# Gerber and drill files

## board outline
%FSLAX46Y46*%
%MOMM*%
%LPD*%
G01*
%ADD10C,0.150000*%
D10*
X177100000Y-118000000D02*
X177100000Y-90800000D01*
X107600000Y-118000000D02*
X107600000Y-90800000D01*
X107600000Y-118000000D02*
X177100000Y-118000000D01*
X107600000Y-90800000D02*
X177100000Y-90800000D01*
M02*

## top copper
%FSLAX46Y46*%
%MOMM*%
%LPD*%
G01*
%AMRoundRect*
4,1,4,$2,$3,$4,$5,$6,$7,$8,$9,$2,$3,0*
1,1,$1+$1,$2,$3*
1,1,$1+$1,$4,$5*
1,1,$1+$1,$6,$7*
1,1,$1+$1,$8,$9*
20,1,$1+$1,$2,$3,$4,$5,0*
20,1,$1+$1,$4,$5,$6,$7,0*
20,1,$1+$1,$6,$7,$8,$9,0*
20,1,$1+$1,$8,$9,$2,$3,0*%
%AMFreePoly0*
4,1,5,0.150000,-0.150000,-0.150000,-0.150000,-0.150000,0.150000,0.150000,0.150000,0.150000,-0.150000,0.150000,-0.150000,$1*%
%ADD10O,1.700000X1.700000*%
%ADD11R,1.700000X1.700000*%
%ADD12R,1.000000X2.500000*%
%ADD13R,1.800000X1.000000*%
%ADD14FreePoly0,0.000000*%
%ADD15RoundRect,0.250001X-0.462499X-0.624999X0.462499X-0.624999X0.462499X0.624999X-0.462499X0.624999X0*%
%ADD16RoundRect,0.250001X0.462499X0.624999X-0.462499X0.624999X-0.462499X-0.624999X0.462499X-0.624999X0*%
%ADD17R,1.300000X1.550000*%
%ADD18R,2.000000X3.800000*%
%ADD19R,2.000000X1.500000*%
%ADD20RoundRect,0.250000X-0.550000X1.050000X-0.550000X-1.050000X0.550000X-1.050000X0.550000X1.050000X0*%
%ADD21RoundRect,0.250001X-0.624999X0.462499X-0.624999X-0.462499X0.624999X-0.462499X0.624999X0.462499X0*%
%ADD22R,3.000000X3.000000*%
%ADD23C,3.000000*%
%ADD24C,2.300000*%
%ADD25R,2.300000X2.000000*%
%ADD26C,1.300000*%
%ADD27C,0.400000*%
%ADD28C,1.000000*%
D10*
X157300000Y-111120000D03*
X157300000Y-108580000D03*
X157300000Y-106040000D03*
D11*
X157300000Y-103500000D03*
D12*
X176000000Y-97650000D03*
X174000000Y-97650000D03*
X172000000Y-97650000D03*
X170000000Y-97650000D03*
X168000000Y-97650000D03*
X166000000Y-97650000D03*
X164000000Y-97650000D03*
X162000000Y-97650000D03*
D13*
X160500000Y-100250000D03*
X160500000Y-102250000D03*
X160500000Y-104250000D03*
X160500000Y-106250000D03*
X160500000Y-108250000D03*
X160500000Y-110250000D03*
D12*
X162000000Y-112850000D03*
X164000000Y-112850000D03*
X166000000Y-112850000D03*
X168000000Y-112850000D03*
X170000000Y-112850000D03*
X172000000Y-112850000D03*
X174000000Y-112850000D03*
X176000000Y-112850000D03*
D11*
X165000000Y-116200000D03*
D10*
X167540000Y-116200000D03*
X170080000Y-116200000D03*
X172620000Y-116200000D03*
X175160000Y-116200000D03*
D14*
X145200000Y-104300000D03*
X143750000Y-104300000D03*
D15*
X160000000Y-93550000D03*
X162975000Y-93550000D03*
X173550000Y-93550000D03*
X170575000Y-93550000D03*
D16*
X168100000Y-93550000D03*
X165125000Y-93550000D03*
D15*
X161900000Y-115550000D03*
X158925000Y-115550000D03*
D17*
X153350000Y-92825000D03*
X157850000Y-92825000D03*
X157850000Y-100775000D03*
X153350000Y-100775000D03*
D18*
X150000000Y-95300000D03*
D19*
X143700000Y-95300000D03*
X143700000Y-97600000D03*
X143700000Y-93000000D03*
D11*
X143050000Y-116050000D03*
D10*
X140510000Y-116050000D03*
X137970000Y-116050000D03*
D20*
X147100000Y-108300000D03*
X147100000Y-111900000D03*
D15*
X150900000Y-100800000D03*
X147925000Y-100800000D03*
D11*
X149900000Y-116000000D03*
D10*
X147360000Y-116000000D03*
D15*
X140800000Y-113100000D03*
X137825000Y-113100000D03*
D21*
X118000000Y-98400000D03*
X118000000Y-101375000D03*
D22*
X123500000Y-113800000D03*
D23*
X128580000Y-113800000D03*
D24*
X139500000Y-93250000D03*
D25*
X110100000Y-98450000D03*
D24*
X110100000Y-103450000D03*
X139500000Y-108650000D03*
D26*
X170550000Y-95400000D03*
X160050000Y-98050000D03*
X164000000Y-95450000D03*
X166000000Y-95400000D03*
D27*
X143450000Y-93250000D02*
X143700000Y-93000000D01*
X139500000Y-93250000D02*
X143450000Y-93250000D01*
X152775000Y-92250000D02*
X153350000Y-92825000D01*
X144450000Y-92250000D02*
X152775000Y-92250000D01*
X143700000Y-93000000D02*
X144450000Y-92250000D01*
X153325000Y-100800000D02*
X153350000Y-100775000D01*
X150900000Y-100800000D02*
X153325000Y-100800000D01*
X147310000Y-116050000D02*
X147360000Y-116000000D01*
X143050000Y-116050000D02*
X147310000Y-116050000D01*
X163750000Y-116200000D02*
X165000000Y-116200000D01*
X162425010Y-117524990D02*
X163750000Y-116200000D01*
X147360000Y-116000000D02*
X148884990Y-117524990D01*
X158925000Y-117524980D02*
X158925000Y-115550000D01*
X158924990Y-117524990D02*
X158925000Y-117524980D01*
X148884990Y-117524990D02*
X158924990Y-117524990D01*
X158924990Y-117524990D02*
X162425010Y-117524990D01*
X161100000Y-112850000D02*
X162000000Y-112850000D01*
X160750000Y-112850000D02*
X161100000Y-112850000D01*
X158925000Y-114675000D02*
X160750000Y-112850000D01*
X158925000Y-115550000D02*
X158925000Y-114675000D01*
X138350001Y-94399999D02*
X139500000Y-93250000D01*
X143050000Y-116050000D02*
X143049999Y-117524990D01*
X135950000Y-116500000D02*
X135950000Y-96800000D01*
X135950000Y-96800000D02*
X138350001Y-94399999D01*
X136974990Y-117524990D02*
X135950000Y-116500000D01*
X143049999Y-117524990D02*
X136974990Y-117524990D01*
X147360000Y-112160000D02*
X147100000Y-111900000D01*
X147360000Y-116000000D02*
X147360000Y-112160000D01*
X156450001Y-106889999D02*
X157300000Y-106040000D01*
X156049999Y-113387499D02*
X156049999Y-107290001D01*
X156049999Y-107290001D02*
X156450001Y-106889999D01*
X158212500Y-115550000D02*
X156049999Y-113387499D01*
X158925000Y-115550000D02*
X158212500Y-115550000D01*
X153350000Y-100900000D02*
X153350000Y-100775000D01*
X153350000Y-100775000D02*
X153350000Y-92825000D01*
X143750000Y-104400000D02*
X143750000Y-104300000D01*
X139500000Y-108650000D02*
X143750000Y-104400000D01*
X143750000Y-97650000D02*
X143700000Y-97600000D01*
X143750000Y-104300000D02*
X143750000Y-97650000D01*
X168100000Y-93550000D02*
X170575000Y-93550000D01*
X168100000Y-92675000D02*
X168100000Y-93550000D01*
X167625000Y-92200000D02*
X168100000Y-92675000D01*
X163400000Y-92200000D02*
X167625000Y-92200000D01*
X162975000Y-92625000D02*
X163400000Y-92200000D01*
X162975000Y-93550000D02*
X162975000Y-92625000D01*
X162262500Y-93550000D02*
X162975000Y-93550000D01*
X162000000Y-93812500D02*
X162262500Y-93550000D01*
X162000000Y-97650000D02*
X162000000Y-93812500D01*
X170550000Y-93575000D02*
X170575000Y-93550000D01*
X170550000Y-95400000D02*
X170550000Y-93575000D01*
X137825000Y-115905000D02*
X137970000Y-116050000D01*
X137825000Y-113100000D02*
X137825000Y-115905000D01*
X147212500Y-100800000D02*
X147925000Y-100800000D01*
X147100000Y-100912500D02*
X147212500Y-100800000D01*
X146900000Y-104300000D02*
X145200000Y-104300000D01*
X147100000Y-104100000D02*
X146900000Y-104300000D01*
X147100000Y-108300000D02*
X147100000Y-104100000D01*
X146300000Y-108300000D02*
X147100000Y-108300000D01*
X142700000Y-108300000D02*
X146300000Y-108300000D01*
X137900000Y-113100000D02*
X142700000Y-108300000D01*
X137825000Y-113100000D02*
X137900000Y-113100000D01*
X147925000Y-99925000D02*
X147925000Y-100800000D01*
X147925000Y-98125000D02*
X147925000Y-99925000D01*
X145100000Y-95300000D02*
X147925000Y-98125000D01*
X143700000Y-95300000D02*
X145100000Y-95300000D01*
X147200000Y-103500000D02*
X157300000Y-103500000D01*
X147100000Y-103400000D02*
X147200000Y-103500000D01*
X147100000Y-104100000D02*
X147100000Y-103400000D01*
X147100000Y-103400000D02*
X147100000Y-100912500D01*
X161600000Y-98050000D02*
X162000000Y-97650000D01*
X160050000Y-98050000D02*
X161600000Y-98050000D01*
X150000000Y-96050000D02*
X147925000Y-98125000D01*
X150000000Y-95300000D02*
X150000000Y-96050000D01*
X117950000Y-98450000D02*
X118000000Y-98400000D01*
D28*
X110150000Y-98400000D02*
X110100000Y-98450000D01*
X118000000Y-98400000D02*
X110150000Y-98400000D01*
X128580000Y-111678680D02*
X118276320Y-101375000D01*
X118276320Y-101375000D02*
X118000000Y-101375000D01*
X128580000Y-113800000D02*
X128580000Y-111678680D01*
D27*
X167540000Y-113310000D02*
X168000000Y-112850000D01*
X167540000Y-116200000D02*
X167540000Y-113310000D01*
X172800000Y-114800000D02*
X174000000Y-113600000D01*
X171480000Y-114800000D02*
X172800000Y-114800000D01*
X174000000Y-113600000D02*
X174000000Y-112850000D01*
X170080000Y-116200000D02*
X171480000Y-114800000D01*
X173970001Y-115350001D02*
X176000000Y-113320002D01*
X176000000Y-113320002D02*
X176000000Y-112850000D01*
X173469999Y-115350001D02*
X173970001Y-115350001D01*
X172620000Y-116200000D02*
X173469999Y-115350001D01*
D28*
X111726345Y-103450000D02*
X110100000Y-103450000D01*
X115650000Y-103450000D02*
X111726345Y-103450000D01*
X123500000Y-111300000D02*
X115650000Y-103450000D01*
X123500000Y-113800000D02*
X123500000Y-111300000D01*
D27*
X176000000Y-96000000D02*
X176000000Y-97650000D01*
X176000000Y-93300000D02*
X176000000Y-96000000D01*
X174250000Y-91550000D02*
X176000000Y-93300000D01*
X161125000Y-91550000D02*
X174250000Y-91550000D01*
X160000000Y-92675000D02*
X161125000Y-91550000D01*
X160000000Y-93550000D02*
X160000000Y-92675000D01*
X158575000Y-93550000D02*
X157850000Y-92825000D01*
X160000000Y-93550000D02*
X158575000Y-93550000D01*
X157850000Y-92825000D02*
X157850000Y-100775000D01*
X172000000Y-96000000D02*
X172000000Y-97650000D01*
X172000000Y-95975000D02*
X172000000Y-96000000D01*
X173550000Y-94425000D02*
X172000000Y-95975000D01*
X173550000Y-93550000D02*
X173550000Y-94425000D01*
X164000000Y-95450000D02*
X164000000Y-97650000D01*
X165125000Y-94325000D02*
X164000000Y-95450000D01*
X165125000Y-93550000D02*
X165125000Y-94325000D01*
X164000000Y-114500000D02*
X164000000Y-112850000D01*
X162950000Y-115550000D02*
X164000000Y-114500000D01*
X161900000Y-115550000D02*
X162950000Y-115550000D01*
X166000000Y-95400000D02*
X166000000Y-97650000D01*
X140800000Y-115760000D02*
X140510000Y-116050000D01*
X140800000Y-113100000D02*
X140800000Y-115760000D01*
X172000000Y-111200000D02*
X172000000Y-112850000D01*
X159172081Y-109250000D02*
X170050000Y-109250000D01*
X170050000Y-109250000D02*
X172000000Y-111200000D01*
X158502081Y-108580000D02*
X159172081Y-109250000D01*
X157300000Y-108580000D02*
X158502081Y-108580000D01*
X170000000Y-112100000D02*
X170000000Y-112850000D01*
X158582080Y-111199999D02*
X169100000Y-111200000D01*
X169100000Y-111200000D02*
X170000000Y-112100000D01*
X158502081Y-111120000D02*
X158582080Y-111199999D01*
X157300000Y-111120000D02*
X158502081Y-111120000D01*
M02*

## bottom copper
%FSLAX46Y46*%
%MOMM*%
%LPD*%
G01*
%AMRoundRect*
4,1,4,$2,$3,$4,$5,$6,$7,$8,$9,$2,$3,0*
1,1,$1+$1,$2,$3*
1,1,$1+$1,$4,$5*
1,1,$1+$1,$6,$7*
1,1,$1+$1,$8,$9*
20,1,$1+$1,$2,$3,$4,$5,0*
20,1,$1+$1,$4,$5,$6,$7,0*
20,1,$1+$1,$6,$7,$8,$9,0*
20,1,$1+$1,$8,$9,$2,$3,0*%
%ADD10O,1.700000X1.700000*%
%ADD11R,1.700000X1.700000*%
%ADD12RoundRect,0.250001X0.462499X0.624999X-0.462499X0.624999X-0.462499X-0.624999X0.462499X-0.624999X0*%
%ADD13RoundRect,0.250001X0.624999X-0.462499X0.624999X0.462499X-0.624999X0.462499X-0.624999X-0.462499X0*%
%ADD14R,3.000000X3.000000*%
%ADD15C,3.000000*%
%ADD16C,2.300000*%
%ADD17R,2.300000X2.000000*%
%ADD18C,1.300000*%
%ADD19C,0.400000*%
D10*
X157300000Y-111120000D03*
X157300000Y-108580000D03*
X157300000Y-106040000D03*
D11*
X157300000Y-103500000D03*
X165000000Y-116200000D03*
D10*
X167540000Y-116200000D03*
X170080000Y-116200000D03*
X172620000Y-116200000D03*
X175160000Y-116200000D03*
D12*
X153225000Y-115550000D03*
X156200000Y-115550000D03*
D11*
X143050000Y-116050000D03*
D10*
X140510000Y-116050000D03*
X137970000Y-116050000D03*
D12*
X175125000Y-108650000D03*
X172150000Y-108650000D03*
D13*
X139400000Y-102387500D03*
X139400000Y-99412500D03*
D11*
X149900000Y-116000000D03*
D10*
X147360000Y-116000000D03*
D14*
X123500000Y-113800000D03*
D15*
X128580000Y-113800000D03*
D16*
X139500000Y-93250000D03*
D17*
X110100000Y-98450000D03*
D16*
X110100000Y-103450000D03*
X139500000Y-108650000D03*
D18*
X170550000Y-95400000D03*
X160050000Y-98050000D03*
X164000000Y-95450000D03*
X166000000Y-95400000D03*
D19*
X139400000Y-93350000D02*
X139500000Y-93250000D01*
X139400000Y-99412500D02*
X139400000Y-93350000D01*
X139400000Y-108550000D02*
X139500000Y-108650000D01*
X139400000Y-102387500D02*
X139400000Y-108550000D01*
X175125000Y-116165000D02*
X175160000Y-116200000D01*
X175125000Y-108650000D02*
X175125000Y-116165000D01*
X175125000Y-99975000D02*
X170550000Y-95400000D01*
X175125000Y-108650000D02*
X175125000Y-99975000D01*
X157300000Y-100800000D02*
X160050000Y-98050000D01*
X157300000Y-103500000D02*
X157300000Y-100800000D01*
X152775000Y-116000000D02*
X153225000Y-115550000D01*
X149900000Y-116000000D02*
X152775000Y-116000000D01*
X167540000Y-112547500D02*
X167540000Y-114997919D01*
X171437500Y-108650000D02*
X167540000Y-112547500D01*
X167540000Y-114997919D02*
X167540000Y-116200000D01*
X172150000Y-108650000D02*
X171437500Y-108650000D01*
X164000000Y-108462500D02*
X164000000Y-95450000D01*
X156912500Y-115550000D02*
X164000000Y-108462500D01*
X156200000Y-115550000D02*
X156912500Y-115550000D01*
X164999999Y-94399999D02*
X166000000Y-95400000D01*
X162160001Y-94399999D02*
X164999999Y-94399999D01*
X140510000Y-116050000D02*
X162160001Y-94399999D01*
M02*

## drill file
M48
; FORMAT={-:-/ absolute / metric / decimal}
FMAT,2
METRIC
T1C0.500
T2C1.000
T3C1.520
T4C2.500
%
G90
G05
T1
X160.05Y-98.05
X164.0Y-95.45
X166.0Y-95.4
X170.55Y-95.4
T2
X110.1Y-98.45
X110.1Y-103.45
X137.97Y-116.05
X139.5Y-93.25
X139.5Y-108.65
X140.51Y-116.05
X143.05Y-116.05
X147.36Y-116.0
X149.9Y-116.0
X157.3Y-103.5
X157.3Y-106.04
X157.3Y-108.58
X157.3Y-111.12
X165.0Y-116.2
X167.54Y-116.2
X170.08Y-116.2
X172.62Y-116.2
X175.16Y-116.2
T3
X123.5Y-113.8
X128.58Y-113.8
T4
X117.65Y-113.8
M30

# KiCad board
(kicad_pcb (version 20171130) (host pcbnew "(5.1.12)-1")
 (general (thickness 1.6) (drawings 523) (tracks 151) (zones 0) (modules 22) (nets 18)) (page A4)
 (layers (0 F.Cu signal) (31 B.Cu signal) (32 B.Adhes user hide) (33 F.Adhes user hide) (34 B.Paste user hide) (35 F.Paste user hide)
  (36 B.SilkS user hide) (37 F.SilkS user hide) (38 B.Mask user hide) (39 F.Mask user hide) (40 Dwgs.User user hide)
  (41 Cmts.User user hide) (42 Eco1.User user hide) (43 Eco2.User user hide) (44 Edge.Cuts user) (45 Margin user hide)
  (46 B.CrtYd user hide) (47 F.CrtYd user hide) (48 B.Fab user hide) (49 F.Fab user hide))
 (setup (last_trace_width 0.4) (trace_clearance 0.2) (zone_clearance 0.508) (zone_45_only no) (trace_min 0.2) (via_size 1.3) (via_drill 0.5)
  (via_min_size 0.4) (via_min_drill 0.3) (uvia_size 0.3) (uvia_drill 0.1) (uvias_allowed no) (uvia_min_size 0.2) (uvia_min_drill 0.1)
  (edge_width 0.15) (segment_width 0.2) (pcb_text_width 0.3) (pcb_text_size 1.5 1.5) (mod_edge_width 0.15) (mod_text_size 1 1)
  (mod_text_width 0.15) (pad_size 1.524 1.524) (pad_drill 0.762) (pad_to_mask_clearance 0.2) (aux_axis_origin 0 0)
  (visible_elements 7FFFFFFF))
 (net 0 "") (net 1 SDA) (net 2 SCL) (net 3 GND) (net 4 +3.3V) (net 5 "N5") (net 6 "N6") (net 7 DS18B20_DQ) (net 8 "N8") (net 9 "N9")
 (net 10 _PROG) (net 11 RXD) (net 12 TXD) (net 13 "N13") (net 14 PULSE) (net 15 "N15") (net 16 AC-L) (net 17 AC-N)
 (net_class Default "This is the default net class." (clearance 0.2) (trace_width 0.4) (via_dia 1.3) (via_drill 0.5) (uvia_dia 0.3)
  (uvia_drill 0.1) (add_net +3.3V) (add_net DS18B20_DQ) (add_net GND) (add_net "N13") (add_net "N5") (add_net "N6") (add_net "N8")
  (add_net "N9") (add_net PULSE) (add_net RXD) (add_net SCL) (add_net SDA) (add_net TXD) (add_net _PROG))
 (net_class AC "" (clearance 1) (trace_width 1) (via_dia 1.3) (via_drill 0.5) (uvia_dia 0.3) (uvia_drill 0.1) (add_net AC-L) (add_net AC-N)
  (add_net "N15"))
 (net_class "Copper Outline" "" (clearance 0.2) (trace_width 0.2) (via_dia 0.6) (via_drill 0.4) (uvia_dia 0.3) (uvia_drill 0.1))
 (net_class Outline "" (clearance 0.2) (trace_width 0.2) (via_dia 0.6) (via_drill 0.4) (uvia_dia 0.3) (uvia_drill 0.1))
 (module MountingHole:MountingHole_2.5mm (layer F.Cu) (at 117.65 113.8)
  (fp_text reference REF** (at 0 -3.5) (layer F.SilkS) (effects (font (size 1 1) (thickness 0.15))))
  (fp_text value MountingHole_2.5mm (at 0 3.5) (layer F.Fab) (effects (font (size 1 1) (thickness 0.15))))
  (pad 1 np_thru_hole circle (at 0 0) (size 2.5 2.5) (drill 2.5) (layers *.Cu *.Mask)))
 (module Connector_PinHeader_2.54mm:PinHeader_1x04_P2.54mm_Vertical (layer F.Cu) (at 157.3 103.5)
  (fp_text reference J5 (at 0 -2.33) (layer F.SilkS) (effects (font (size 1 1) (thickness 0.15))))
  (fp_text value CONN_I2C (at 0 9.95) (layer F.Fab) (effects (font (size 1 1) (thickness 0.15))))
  (pad 4 thru_hole oval (at 0 7.62) (size 1.7 1.7) (drill 1) (layers *.Cu *.Mask) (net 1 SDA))
  (pad 3 thru_hole oval (at 0 5.08) (size 1.7 1.7) (drill 1) (layers *.Cu *.Mask) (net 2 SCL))
  (pad 2 thru_hole oval (at 0 2.54) (size 1.7 1.7) (drill 1) (layers *.Cu *.Mask) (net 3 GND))
  (pad 1 thru_hole rect (at 0 0) (size 1.7 1.7) (drill 1) (layers *.Cu *.Mask) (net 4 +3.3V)))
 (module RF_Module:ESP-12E (layer F.Cu) (at 172.5 105.25 270)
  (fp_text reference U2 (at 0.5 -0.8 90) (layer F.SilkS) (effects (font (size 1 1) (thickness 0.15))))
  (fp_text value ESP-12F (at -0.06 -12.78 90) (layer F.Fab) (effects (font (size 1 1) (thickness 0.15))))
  (pad 1 smd rect (at -7.6 -3.5 270) (size 2.5 1) (layers F.Cu F.Paste F.Mask) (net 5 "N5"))
  (pad 2 smd rect (at -7.6 -1.5 270) (size 2.5 1) (layers F.Cu F.Paste F.Mask))
  (pad 3 smd rect (at -7.6 0.5 270) (size 2.5 1) (layers F.Cu F.Paste F.Mask) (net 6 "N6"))
  (pad 4 smd rect (at -7.6 2.5 270) (size 2.5 1) (layers F.Cu F.Paste F.Mask))
  (pad 5 smd rect (at -7.6 4.5 270) (size 2.5 1) (layers F.Cu F.Paste F.Mask))
  (pad 6 smd rect (at -7.6 6.5 270) (size 2.5 1) (layers F.Cu F.Paste F.Mask) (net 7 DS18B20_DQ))
  (pad 7 smd rect (at -7.6 8.5 270) (size 2.5 1) (layers F.Cu F.Paste F.Mask) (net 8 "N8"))
  (pad 8 smd rect (at -7.6 10.5 270) (size 2.5 1) (layers F.Cu F.Paste F.Mask) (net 4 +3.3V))
  (pad 9 smd rect (at -5 12 270) (size 1 1.8) (layers F.Cu F.Paste F.Mask))
  (pad 10 smd rect (at -3 12 270) (size 1 1.8) (layers F.Cu F.Paste F.Mask))
  (pad 11 smd rect (at -1 12 270) (size 1 1.8) (layers F.Cu F.Paste F.Mask))
  (pad 12 smd rect (at 1 12 270) (size 1 1.8) (layers F.Cu F.Paste F.Mask))
  (pad 13 smd rect (at 3 12 270) (size 1 1.8) (layers F.Cu F.Paste F.Mask))
  (pad 14 smd rect (at 5 12 270) (size 1 1.8) (layers F.Cu F.Paste F.Mask))
  (pad 15 smd rect (at 7.6 10.5 270) (size 2.5 1) (layers F.Cu F.Paste F.Mask) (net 3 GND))
  (pad 16 smd rect (at 7.6 8.5 270) (size 2.5 1) (layers F.Cu F.Paste F.Mask) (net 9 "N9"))
  (pad 17 smd rect (at 7.6 6.5 270) (size 2.5 1) (layers F.Cu F.Paste F.Mask))
  (pad 18 smd rect (at 7.6 4.5 270) (size 2.5 1) (layers F.Cu F.Paste F.Mask) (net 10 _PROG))
  (pad 19 smd rect (at 7.6 2.5 270) (size 2.5 1) (layers F.Cu F.Paste F.Mask) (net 1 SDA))
  (pad 20 smd rect (at 7.6 0.5 270) (size 2.5 1) (layers F.Cu F.Paste F.Mask) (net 2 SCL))
  (pad 21 smd rect (at 7.6 -1.5 270) (size 2.5 1) (layers F.Cu F.Paste F.Mask) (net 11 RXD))
  (pad 22 smd rect (at 7.6 -3.5 270) (size 2.5 1) (layers F.Cu F.Paste F.Mask) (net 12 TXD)))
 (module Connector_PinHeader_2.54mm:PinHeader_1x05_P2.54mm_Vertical (layer F.Cu) (at 165 116.2 90)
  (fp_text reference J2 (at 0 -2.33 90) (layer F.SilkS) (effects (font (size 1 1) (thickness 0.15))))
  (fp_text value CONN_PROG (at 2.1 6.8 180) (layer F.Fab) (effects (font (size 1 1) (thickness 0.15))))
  (pad 1 thru_hole rect (at 0 0 90) (size 1.7 1.7) (drill 1) (layers *.Cu *.Mask) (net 3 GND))
  (pad 2 thru_hole oval (at 0 2.54 90) (size 1.7 1.7) (drill 1) (layers *.Cu *.Mask) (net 10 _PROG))
  (pad 3 thru_hole oval (at 0 5.08 90) (size 1.7 1.7) (drill 1) (layers *.Cu *.Mask) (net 11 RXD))
  (pad 4 thru_hole oval (at 0 7.62 90) (size 1.7 1.7) (drill 1) (layers *.Cu *.Mask) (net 12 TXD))
  (pad 5 thru_hole oval (at 0 10.16 90) (size 1.7 1.7) (drill 1) (layers *.Cu *.Mask) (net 4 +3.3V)))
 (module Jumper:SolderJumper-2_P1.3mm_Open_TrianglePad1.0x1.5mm (layer F.Cu) (at 144.475 104.3)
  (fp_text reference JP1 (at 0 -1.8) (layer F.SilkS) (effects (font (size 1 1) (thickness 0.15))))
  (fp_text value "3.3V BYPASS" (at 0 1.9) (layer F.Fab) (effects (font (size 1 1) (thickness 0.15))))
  (pad 2 smd custom (at 0.725 0) (size 0.3 0.3) (layers F.Cu F.Mask) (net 4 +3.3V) (zone_connect 2)
   (options (clearance outline) (anchor rect)) (primitives))
  (pad 1 smd custom (at -0.725 0) (size 0.3 0.3) (layers F.Cu F.Mask) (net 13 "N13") (zone_connect 2)
   (options (clearance outline) (anchor rect)) (primitives)))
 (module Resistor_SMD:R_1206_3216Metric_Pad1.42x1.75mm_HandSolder (layer F.Cu) (at 161.4875 93.55)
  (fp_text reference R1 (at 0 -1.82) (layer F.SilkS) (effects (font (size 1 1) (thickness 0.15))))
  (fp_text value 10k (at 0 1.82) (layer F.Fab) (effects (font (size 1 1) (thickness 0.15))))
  (pad 1 smd roundrect (at -1.4875 0) (size 1.425 1.75) (layers F.Cu F.Paste F.Mask) (roundrect_rratio 0.175439) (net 5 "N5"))
  (pad 2 smd roundrect (at 1.4875 0) (size 1.425 1.75) (layers F.Cu F.Paste F.Mask) (roundrect_rratio 0.175439) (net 4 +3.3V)))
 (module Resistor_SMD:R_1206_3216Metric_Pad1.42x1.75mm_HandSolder (layer F.Cu) (at 172.0625 93.55)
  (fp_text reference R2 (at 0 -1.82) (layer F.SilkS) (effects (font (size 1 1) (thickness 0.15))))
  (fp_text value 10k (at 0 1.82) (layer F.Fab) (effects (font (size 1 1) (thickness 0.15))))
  (pad 2 smd roundrect (at 1.4875 0) (size 1.425 1.75) (layers F.Cu F.Paste F.Mask) (roundrect_rratio 0.175439) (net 6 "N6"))
  (pad 1 smd roundrect (at -1.4875 0) (size 1.425 1.75) (layers F.Cu F.Paste F.Mask) (roundrect_rratio 0.175439) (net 4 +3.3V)))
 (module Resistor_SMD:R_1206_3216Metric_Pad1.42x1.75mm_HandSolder (layer B.Cu) (at 154.7125 115.55 180)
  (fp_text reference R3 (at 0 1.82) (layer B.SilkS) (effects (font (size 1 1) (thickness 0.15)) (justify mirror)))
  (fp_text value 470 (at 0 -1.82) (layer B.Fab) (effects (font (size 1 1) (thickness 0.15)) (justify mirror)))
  (pad 2 smd roundrect (at 1.4875 0 180) (size 1.425 1.75) (layers B.Cu B.Paste B.Mask) (roundrect_rratio 0.175439) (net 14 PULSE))
  (pad 1 smd roundrect (at -1.4875 0 180) (size 1.425 1.75) (layers B.Cu B.Paste B.Mask) (roundrect_rratio 0.175439) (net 8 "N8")))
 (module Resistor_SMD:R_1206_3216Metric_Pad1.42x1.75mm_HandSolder (layer F.Cu) (at 166.6125 93.55 180)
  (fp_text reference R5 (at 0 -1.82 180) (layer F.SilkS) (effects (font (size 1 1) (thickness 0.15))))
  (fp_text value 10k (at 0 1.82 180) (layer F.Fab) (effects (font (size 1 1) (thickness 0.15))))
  (pad 1 smd roundrect (at -1.4875 0 180) (size 1.425 1.75) (layers F.Cu F.Paste F.Mask) (roundrect_rratio 0.175439) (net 4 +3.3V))
  (pad 2 smd roundrect (at 1.4875 0 180) (size 1.425 1.75) (layers F.Cu F.Paste F.Mask) (roundrect_rratio 0.175439) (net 8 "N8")))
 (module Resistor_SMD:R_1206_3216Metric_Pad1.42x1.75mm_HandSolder (layer F.Cu) (at 160.4125 115.55)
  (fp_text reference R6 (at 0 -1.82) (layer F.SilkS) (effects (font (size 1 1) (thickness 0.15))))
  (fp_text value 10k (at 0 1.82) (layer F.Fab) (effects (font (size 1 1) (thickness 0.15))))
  (pad 2 smd roundrect (at 1.4875 0) (size 1.425 1.75) (layers F.Cu F.Paste F.Mask) (roundrect_rratio 0.175439) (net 9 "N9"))
  (pad 1 smd roundrect (at -1.4875 0) (size 1.425 1.75) (layers F.Cu F.Paste F.Mask) (roundrect_rratio 0.175439) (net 3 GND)))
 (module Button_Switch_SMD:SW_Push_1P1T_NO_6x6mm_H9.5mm (layer F.Cu) (at 155.6 96.8 270)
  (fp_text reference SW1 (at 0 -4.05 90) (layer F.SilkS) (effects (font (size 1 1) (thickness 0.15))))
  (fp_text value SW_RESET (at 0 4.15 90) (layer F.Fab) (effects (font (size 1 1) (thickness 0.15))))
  (pad 2 smd rect (at -3.975 2.25 270) (size 1.55 1.3) (layers F.Cu F.Paste F.Mask) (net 3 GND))
  (pad 1 smd rect (at -3.975 -2.25 270) (size 1.55 1.3) (layers F.Cu F.Paste F.Mask) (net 5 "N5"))
  (pad 1 smd rect (at 3.975 -2.25 270) (size 1.55 1.3) (layers F.Cu F.Paste F.Mask) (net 5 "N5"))
  (pad 2 smd rect (at 3.975 2.25 270) (size 1.55 1.3) (layers F.Cu F.Paste F.Mask) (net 3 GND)))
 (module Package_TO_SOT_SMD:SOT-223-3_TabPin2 (layer F.Cu) (at 146.85 95.3)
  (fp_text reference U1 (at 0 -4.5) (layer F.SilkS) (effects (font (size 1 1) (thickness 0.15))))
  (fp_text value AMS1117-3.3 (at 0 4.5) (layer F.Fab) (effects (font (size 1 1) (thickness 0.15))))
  (pad 2 smd rect (at 3.15 0) (size 2 3.8) (layers F.Cu F.Paste F.Mask) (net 4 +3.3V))
  (pad 2 smd rect (at -3.15 0) (size 2 1.5) (layers F.Cu F.Paste F.Mask) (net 4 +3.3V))
  (pad 3 smd rect (at -3.15 2.3) (size 2 1.5) (layers F.Cu F.Paste F.Mask) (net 13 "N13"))
  (pad 1 smd rect (at -3.15 -2.3) (size 2 1.5) (layers F.Cu F.Paste F.Mask) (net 3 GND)))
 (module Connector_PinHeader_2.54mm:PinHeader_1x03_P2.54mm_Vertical (layer F.Cu) (at 143.05 116.05 270)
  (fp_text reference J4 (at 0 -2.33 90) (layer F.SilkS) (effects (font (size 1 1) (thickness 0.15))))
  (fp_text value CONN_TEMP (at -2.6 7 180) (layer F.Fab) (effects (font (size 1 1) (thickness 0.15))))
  (pad 1 thru_hole rect (at 0 0 270) (size 1.7 1.7) (drill 1) (layers *.Cu *.Mask) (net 3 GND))
  (pad 2 thru_hole oval (at 0 2.54 270) (size 1.7 1.7) (drill 1) (layers *.Cu *.Mask) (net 7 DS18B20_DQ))
  (pad 3 thru_hole oval (at 0 5.08 270) (size 1.7 1.7) (drill 1) (layers *.Cu *.Mask) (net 4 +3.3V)))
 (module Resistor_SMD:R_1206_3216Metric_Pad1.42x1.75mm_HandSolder (layer B.Cu) (at 173.6375 108.65 180)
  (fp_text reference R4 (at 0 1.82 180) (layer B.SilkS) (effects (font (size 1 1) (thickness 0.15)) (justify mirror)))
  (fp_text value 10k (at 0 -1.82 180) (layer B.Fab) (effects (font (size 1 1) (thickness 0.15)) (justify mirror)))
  (pad 1 smd roundrect (at -1.4875 0 180) (size 1.425 1.75) (layers B.Cu B.Paste B.Mask) (roundrect_rratio 0.175439) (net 4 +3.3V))
  (pad 2 smd roundrect (at 1.4875 0 180) (size 1.425 1.75) (layers B.Cu B.Paste B.Mask) (roundrect_rratio 0.175439) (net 10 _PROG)))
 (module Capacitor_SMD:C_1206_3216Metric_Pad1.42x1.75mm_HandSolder (layer B.Cu) (at 139.4 100.9 90)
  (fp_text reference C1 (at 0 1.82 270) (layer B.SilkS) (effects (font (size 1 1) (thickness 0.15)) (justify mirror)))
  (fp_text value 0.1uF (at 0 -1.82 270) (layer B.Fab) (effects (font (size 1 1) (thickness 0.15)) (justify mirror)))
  (pad 1 smd roundrect (at -1.4875 0 90) (size 1.425 1.75) (layers B.Cu B.Paste B.Mask) (roundrect_rratio 0.175439) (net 13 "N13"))
  (pad 2 smd roundrect (at 1.4875 0 90) (size 1.425 1.75) (layers B.Cu B.Paste B.Mask) (roundrect_rratio 0.175439) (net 3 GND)))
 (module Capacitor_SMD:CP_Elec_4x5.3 (layer F.Cu) (at 147.1 110.1 270)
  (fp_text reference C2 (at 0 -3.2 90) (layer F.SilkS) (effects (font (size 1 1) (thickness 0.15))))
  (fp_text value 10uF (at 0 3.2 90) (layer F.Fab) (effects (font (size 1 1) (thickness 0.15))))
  (pad 1 smd roundrect (at -1.8 0 270) (size 2.6 1.6) (layers F.Cu F.Paste F.Mask) (roundrect_rratio 0.15625) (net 4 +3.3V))
  (pad 2 smd roundrect (at 1.8 0 270) (size 2.6 1.6) (layers F.Cu F.Paste F.Mask) (roundrect_rratio 0.15625) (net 3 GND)))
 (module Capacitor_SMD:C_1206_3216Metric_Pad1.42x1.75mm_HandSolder (layer F.Cu) (at 149.4125 100.8)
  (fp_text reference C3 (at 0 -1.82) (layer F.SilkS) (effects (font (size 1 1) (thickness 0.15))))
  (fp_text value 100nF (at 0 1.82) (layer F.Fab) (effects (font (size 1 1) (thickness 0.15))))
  (pad 2 smd roundrect (at 1.4875 0) (size 1.425 1.75) (layers F.Cu F.Paste F.Mask) (roundrect_rratio 0.175439) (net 3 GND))
  (pad 1 smd roundrect (at -1.4875 0) (size 1.425 1.75) (layers F.Cu F.Paste F.Mask) (roundrect_rratio 0.175439) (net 4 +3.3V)))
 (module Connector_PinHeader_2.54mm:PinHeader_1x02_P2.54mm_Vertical (layer F.Cu) (at 149.9 116 270)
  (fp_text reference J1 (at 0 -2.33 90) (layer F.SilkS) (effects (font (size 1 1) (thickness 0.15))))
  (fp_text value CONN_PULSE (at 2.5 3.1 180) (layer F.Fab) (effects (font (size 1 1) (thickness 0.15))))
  (pad 1 thru_hole rect (at 0 0 270) (size 1.7 1.7) (drill 1) (layers *.Cu *.Mask) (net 14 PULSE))
  (pad 2 thru_hole oval (at 0 2.54 270) (size 1.7 1.7) (drill 1) (layers *.Cu *.Mask) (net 3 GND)))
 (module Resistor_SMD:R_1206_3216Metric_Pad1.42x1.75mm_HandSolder (layer F.Cu) (at 139.3125 113.1)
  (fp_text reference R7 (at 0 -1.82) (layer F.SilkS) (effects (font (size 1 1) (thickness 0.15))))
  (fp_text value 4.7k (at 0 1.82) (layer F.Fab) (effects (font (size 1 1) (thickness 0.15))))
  (pad 2 smd roundrect (at 1.4875 0) (size 1.425 1.75) (layers F.Cu F.Paste F.Mask) (roundrect_rratio 0.175439) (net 7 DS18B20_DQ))
  (pad 1 smd roundrect (at -1.4875 0) (size 1.425 1.75) (layers F.Cu F.Paste F.Mask) (roundrect_rratio 0.175439) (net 4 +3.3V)))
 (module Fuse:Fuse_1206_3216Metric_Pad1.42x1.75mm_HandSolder (layer F.Cu) (at 118 99.8875 270)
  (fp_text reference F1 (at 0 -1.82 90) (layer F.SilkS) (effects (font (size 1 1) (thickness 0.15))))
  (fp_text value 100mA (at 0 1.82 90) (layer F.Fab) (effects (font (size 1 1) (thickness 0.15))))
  (pad 1 smd roundrect (at -1.4875 0 270) (size 1.425 1.75) (layers F.Cu F.Paste F.Mask) (roundrect_rratio 0.175439) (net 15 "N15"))
  (pad 2 smd roundrect (at 1.4875 0 270) (size 1.425 1.75) (layers F.Cu F.Paste F.Mask) (roundrect_rratio 0.175439) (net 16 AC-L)))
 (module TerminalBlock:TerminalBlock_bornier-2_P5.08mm (layer F.Cu) (at 123.5 113.8)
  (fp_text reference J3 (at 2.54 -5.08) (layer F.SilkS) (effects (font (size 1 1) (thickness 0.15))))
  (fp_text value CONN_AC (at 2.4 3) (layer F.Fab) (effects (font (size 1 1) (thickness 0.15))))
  (pad 1 thru_hole rect (at 0 0) (size 3 3) (drill 1.52) (layers *.Cu *.Mask) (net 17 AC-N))
  (pad 2 thru_hole circle (at 5.08 0) (size 3 3) (drill 1.52) (layers *.Cu *.Mask) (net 16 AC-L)))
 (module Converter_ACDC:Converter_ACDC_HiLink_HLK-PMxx (layer F.Cu) (at 110.1 98.45)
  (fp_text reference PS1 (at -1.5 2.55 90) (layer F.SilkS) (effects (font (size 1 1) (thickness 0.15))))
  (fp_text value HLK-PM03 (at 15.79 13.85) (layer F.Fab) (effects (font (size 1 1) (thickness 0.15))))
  (pad 3 thru_hole circle (at 29.4 -5.2) (size 2.3 2.3) (drill 1) (layers *.Cu *.Mask) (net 3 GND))
  (pad 1 thru_hole rect (at 0 0) (size 2.3 2) (drill 1) (layers *.Cu *.Mask) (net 15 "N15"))
  (pad 2 thru_hole circle (at 0 5) (size 2.3 2.3) (drill 1) (layers *.Cu *.Mask) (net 17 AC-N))
  (pad 4 thru_hole circle (at 29.4 10.2) (size 2.3 2.3) (drill 1) (layers *.Cu *.Mask) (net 13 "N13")))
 (gr_line (start 177.1 118) (end 177.1 90.8) (layer Edge.Cuts) (width 0.15))
 (gr_line (start 107.6 118) (end 107.6 90.8) (layer Edge.Cuts) (width 0.15))
 (gr_line (start 107.6 118) (end 177.1 118) (layer Edge.Cuts) (width 0.15))
 (gr_line (start 107.6 90.8) (end 177.1 90.8) (layer Edge.Cuts) (width 0.15))
 (segment (start 143.45 93.25) (end 143.7 93) (width 0.4) (layer F.Cu) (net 3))
 (segment (start 139.5 93.25) (end 143.45 93.25) (width 0.4) (layer F.Cu) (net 3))
 (segment (start 152.775 92.25) (end 153.35 92.825) (width 0.4) (layer F.Cu) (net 3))
 (segment (start 144.45 92.25) (end 152.775 92.25) (width 0.4) (layer F.Cu) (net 3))
 (segment (start 143.7 93) (end 144.45 92.25) (width 0.4) (layer F.Cu) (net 3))
 (segment (start 153.325 100.8) (end 153.35 100.775) (width 0.4) (layer F.Cu) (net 3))
 (segment (start 150.9 100.8) (end 153.325 100.8) (width 0.4) (layer F.Cu) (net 3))
 (segment (start 147.31 116.05) (end 147.36 116) (width 0.4) (layer F.Cu) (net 3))
 (segment (start 143.05 116.05) (end 147.31 116.05) (width 0.4) (layer F.Cu) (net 3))
 (segment (start 163.75 116.2) (end 165 116.2) (width 0.4) (layer F.Cu) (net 3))
 (segment (start 162.42501 117.52499) (end 163.75 116.2) (width 0.4) (layer F.Cu) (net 3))
 (segment (start 147.36 116) (end 148.88499 117.52499) (width 0.4) (layer F.Cu) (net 3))
 (segment (start 158.925 117.52498) (end 158.925 115.55) (width 0.4) (layer F.Cu) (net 3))
 (segment (start 158.92499 117.52499) (end 158.925 117.52498) (width 0.4) (layer F.Cu) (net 3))
 (segment (start 148.88499 117.52499) (end 158.92499 117.52499) (width 0.4) (layer F.Cu) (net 3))
 (segment (start 158.92499 117.52499) (end 162.42501 117.52499) (width 0.4) (layer F.Cu) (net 3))
 (segment (start 161.1 112.85) (end 162 112.85) (width 0.4) (layer F.Cu) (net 3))
 (segment (start 160.75 112.85) (end 161.1 112.85) (width 0.4) (layer F.Cu) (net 3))
 (segment (start 158.925 114.675) (end 160.75 112.85) (width 0.4) (layer F.Cu) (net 3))
 (segment (start 158.925 115.55) (end 158.925 114.675) (width 0.4) (layer F.Cu) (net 3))
 (segment (start 139.4 93.35) (end 139.5 93.25) (width 0.4) (layer B.Cu) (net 3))
 (segment (start 139.4 99.4125) (end 139.4 93.35) (width 0.4) (layer B.Cu) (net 3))
 (segment (start 138.350001 94.399999) (end 139.5 93.25) (width 0.4) (layer F.Cu) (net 3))
 (segment (start 143.05 116.05) (end 143.049999 117.52499) (width 0.4) (layer F.Cu) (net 3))
 (segment (start 135.95 116.5) (end 135.95 96.8) (width 0.4) (layer F.Cu) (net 3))
 (segment (start 135.95 96.8) (end 138.350001 94.399999) (width 0.4) (layer F.Cu) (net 3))
 (segment (start 136.97499 117.52499) (end 135.95 116.5) (width 0.4) (layer F.Cu) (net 3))
 (segment (start 143.049999 117.52499) (end 136.97499 117.52499) (width 0.4) (layer F.Cu) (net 3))
 (segment (start 147.36 112.16) (end 147.1 111.9) (width 0.4) (layer F.Cu) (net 3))
 (segment (start 147.36 116) (end 147.36 112.16) (width 0.4) (layer F.Cu) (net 3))
 (segment (start 156.450001 106.889999) (end 157.3 106.04) (width 0.4) (layer F.Cu) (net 3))
 (segment (start 156.049999 113.387499) (end 156.049999 107.290001) (width 0.4) (layer F.Cu) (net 3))
 (segment (start 156.049999 107.290001) (end 156.450001 106.889999) (width 0.4) (layer F.Cu) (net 3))
 (segment (start 158.2125 115.55) (end 156.049999 113.387499) (width 0.4) (layer F.Cu) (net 3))
 (segment (start 158.925 115.55) (end 158.2125 115.55) (width 0.4) (layer F.Cu) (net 3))
 (segment (start 153.35 100.9) (end 153.35 100.775) (width 0.4) (layer F.Cu) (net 3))
 (segment (start 153.35 100.775) (end 153.35 92.825) (width 0.4) (layer F.Cu) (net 3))
 (segment (start 143.75 104.4) (end 143.75 104.3) (width 0.4) (layer F.Cu) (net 13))
 (segment (start 139.5 108.65) (end 143.75 104.4) (width 0.4) (layer F.Cu) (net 13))
 (segment (start 139.4 108.55) (end 139.5 108.65) (width 0.4) (layer B.Cu) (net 13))
 (segment (start 139.4 102.3875) (end 139.4 108.55) (width 0.4) (layer B.Cu) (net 13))
 (segment (start 143.75 97.65) (end 143.7 97.6) (width 0.4) (layer F.Cu) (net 13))
 (segment (start 143.75 104.3) (end 143.75 97.65) (width 0.4) (layer F.Cu) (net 13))
 (segment (start 168.1 93.55) (end 170.575 93.55) (width 0.4) (layer F.Cu) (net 4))
 (segment (start 168.1 92.675) (end 168.1 93.55) (width 0.4) (layer F.Cu) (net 4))
 (segment (start 167.625 92.2) (end 168.1 92.675) (width 0.4) (layer F.Cu) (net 4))
 (segment (start 163.4 92.2) (end 167.625 92.2) (width 0.4) (layer F.Cu) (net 4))
 (segment (start 162.975 92.625) (end 163.4 92.2) (width 0.4) (layer F.Cu) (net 4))
 (segment (start 162.975 93.55) (end 162.975 92.625) (width 0.4) (layer F.Cu) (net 4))
 (segment (start 162.2625 93.55) (end 162.975 93.55) (width 0.4) (layer F.Cu) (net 4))
 (segment (start 162 93.8125) (end 162.2625 93.55) (width 0.4) (layer F.Cu) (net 4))
 (segment (start 162 97.65) (end 162 93.8125) (width 0.4) (layer F.Cu) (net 4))
 (segment (start 175.125 116.165) (end 175.16 116.2) (width 0.4) (layer B.Cu) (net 4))
 (segment (start 175.125 108.65) (end 175.125 116.165) (width 0.4) (layer B.Cu) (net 4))
 (segment (start 175.125 99.975) (end 170.55 95.4) (width 0.4) (layer B.Cu) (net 4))
 (segment (start 175.125 108.65) (end 175.125 99.975) (width 0.4) (layer B.Cu) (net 4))
 (segment (start 170.55 93.575) (end 170.575 93.55) (width 0.4) (layer F.Cu) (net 4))
 (segment (start 170.55 95.4) (end 170.55 93.575) (width 0.4) (layer F.Cu) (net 4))
 (segment (start 137.825 115.905) (end 137.97 116.05) (width 0.4) (layer F.Cu) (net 4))
 (segment (start 137.825 113.1) (end 137.825 115.905) (width 0.4) (layer F.Cu) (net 4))
 (segment (start 147.2125 100.8) (end 147.925 100.8) (width 0.4) (layer F.Cu) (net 4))
 (segment (start 147.1 100.9125) (end 147.2125 100.8) (width 0.4) (layer F.Cu) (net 4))
 (segment (start 146.9 104.3) (end 145.2 104.3) (width 0.4) (layer F.Cu) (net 4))
 (segment (start 147.1 104.1) (end 146.9 104.3) (width 0.4) (layer F.Cu) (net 4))
 (segment (start 147.1 108.3) (end 147.1 104.1) (width 0.4) (layer F.Cu) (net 4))
 (segment (start 146.3 108.3) (end 147.1 108.3) (width 0.4) (layer F.Cu) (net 4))
 (segment (start 142.7 108.3) (end 146.3 108.3) (width 0.4) (layer F.Cu) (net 4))
 (segment (start 137.9 113.1) (end 142.7 108.3) (width 0.4) (layer F.Cu) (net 4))
 (segment (start 137.825 113.1) (end 137.9 113.1) (width 0.4) (layer F.Cu) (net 4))
 (segment (start 147.925 99.925) (end 147.925 100.8) (width 0.4) (layer F.Cu) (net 4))
 (segment (start 147.925 98.125) (end 147.925 99.925) (width 0.4) (layer F.Cu) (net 4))
 (segment (start 145.1 95.3) (end 147.925 98.125) (width 0.4) (layer F.Cu) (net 4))
 (segment (start 143.7 95.3) (end 145.1 95.3) (width 0.4) (layer F.Cu) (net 4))
 (segment (start 147.2 103.5) (end 157.3 103.5) (width 0.4) (layer F.Cu) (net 4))
 (segment (start 147.1 103.4) (end 147.2 103.5) (width 0.4) (layer F.Cu) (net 4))
 (segment (start 147.1 104.1) (end 147.1 103.4) (width 0.4) (layer F.Cu) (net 4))
 (segment (start 147.1 103.4) (end 147.1 100.9125) (width 0.4) (layer F.Cu) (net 4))
 (segment (start 157.3 100.8) (end 160.05 98.05) (width 0.4) (layer B.Cu) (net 4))
 (segment (start 157.3 103.5) (end 157.3 100.8) (width 0.4) (layer B.Cu) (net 4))
 (segment (start 161.6 98.05) (end 162 97.65) (width 0.4) (layer F.Cu) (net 4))
 (segment (start 160.05 98.05) (end 161.6 98.05) (width 0.4) (layer F.Cu) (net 4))
 (segment (start 150 96.05) (end 147.925 98.125) (width 0.4) (layer F.Cu) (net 4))
 (segment (start 150 95.3) (end 150 96.05) (width 0.4) (layer F.Cu) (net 4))
 (segment (start 117.95 98.45) (end 118 98.4) (width 0.4) (layer F.Cu) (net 15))
 (segment (start 110.15 98.4) (end 110.1 98.45) (width 1) (layer F.Cu) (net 15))
 (segment (start 118 98.4) (end 110.15 98.4) (width 1) (layer F.Cu) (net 15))
 (segment (start 128.58 111.67868) (end 118.27632 101.375) (width 1) (layer F.Cu) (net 16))
 (segment (start 118.27632 101.375) (end 118 101.375) (width 1) (layer F.Cu) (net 16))
 (segment (start 128.58 113.8) (end 128.58 111.67868) (width 1) (layer F.Cu) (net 16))
 (segment (start 152.775 116) (end 153.225 115.55) (width 0.4) (layer B.Cu) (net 14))
 (segment (start 149.9 116) (end 152.775 116) (width 0.4) (layer B.Cu) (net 14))
 (segment (start 167.54 112.5475) (end 167.54 114.997919) (width 0.4) (layer B.Cu) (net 10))
 (segment (start 171.4375 108.65) (end 167.54 112.5475) (width 0.4) (layer B.Cu) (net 10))
 (segment (start 167.54 114.997919) (end 167.54 116.2) (width 0.4) (layer B.Cu) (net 10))
 (segment (start 172.15 108.65) (end 171.4375 108.65) (width 0.4) (layer B.Cu) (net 10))
 (segment (start 167.54 113.31) (end 168 112.85) (width 0.4) (layer F.Cu) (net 10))
 (segment (start 167.54 116.2) (end 167.54 113.31) (width 0.4) (layer F.Cu) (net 10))
 (segment (start 172.8 114.8) (end 174 113.6) (width 0.4) (layer F.Cu) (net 11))
 (segment (start 171.48 114.8) (end 172.8 114.8) (width 0.4) (layer F.Cu) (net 11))
 (segment (start 174 113.6) (end 174 112.85) (width 0.4) (layer F.Cu) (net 11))
 (segment (start 170.08 116.2) (end 171.48 114.8) (width 0.4) (layer F.Cu) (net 11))
 (segment (start 173.970001 115.350001) (end 176 113.320002) (width 0.4) (layer F.Cu) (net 12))
 (segment (start 176 113.320002) (end 176 112.85) (width 0.4) (layer F.Cu) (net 12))
 (segment (start 173.469999 115.350001) (end 173.970001 115.350001) (width 0.4) (layer F.Cu) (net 12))
 (segment (start 172.62 116.2) (end 173.469999 115.350001) (width 0.4) (layer F.Cu) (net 12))
 (segment (start 111.726345 103.45) (end 110.1 103.45) (width 1) (layer F.Cu) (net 17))
 (segment (start 115.65 103.45) (end 111.726345 103.45) (width 1) (layer F.Cu) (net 17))
 (segment (start 123.5 111.3) (end 115.65 103.45) (width 1) (layer F.Cu) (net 17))
 (segment (start 123.5 113.8) (end 123.5 111.3) (width 1) (layer F.Cu) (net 17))
 (segment (start 176 96) (end 176 97.65) (width 0.4) (layer F.Cu) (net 5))
 (segment (start 176 93.3) (end 176 96) (width 0.4) (layer F.Cu) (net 5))
 (segment (start 174.25 91.55) (end 176 93.3) (width 0.4) (layer F.Cu) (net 5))
 (segment (start 161.125 91.55) (end 174.25 91.55) (width 0.4) (layer F.Cu) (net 5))
 (segment (start 160 92.675) (end 161.125 91.55) (width 0.4) (layer F.Cu) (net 5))
 (segment (start 160 93.55) (end 160 92.675) (width 0.4) (layer F.Cu) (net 5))
 (segment (start 158.575 93.55) (end 157.85 92.825) (width 0.4) (layer F.Cu) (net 5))
 (segment (start 160 93.55) (end 158.575 93.55) (width 0.4) (layer F.Cu) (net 5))
 (segment (start 157.85 92.825) (end 157.85 100.775) (width 0.4) (layer F.Cu) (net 5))
 (segment (start 172 96) (end 172 97.65) (width 0.4) (layer F.Cu) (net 6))
 (segment (start 172 95.975) (end 172 96) (width 0.4) (layer F.Cu) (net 6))
 (segment (start 173.55 94.425) (end 172 95.975) (width 0.4) (layer F.Cu) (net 6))
 (segment (start 173.55 93.55) (end 173.55 94.425) (width 0.4) (layer F.Cu) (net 6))
 (segment (start 164 108.4625) (end 164 95.45) (width 0.4) (layer B.Cu) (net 8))
 (segment (start 156.9125 115.55) (end 164 108.4625) (width 0.4) (layer B.Cu) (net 8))
 (segment (start 156.2 115.55) (end 156.9125 115.55) (width 0.4) (layer B.Cu) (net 8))
 (segment (start 164 95.45) (end 164 97.65) (width 0.4) (layer F.Cu) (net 8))
 (segment (start 165.125 94.325) (end 164 95.45) (width 0.4) (layer F.Cu) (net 8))
 (segment (start 165.125 93.55) (end 165.125 94.325) (width 0.4) (layer F.Cu) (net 8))
 (segment (start 164 114.5) (end 164 112.85) (width 0.4) (layer F.Cu) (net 9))
 (segment (start 162.95 115.55) (end 164 114.5) (width 0.4) (layer F.Cu) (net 9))
 (segment (start 161.9 115.55) (end 162.95 115.55) (width 0.4) (layer F.Cu) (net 9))
 (segment (start 164.999999 94.399999) (end 166 95.4) (width 0.4) (layer B.Cu) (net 7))
 (segment (start 162.160001 94.399999) (end 164.999999 94.399999) (width 0.4) (layer B.Cu) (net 7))
 (segment (start 140.51 116.05) (end 162.160001 94.399999) (width 0.4) (layer B.Cu) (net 7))
 (segment (start 166 95.4) (end 166 97.65) (width 0.4) (layer F.Cu) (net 7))
 (segment (start 140.8 115.76) (end 140.51 116.05) (width 0.4) (layer F.Cu) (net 7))
 (segment (start 140.8 113.1) (end 140.8 115.76) (width 0.4) (layer F.Cu) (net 7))
 (segment (start 172 111.2) (end 172 112.85) (width 0.4) (layer F.Cu) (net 2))
 (segment (start 159.172081 109.25) (end 170.05 109.25) (width 0.4) (layer F.Cu) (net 2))
 (segment (start 170.05 109.25) (end 172 111.2) (width 0.4) (layer F.Cu) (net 2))
 (segment (start 158.502081 108.58) (end 159.172081 109.25) (width 0.4) (layer F.Cu) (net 2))
 (segment (start 157.3 108.58) (end 158.502081 108.58) (width 0.4) (layer F.Cu) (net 2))
 (segment (start 170 112.1) (end 170 112.85) (width 0.4) (layer F.Cu) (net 1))
 (segment (start 158.58208 111.199999) (end 169.1 111.2) (width 0.4) (layer F.Cu) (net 1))
 (segment (start 169.1 111.2) (end 170 112.1) (width 0.4) (layer F.Cu) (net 1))
 (segment (start 158.502081 111.12) (end 158.58208 111.199999) (width 0.4) (layer F.Cu) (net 1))
 (segment (start 157.3 111.12) (end 158.502081 111.12) (width 0.4) (layer F.Cu) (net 1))
 (via (at 170.55 95.4) (size 1.3) (drill 0.5) (layers F.Cu B.Cu) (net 4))
 (via (at 160.05 98.05) (size 1.3) (drill 0.5) (layers F.Cu B.Cu) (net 4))
 (via (at 164 95.45) (size 1.3) (drill 0.5) (layers F.Cu B.Cu) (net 8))
 (via (at 166 95.4) (size 1.3) (drill 0.5) (layers F.Cu B.Cu) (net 7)))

